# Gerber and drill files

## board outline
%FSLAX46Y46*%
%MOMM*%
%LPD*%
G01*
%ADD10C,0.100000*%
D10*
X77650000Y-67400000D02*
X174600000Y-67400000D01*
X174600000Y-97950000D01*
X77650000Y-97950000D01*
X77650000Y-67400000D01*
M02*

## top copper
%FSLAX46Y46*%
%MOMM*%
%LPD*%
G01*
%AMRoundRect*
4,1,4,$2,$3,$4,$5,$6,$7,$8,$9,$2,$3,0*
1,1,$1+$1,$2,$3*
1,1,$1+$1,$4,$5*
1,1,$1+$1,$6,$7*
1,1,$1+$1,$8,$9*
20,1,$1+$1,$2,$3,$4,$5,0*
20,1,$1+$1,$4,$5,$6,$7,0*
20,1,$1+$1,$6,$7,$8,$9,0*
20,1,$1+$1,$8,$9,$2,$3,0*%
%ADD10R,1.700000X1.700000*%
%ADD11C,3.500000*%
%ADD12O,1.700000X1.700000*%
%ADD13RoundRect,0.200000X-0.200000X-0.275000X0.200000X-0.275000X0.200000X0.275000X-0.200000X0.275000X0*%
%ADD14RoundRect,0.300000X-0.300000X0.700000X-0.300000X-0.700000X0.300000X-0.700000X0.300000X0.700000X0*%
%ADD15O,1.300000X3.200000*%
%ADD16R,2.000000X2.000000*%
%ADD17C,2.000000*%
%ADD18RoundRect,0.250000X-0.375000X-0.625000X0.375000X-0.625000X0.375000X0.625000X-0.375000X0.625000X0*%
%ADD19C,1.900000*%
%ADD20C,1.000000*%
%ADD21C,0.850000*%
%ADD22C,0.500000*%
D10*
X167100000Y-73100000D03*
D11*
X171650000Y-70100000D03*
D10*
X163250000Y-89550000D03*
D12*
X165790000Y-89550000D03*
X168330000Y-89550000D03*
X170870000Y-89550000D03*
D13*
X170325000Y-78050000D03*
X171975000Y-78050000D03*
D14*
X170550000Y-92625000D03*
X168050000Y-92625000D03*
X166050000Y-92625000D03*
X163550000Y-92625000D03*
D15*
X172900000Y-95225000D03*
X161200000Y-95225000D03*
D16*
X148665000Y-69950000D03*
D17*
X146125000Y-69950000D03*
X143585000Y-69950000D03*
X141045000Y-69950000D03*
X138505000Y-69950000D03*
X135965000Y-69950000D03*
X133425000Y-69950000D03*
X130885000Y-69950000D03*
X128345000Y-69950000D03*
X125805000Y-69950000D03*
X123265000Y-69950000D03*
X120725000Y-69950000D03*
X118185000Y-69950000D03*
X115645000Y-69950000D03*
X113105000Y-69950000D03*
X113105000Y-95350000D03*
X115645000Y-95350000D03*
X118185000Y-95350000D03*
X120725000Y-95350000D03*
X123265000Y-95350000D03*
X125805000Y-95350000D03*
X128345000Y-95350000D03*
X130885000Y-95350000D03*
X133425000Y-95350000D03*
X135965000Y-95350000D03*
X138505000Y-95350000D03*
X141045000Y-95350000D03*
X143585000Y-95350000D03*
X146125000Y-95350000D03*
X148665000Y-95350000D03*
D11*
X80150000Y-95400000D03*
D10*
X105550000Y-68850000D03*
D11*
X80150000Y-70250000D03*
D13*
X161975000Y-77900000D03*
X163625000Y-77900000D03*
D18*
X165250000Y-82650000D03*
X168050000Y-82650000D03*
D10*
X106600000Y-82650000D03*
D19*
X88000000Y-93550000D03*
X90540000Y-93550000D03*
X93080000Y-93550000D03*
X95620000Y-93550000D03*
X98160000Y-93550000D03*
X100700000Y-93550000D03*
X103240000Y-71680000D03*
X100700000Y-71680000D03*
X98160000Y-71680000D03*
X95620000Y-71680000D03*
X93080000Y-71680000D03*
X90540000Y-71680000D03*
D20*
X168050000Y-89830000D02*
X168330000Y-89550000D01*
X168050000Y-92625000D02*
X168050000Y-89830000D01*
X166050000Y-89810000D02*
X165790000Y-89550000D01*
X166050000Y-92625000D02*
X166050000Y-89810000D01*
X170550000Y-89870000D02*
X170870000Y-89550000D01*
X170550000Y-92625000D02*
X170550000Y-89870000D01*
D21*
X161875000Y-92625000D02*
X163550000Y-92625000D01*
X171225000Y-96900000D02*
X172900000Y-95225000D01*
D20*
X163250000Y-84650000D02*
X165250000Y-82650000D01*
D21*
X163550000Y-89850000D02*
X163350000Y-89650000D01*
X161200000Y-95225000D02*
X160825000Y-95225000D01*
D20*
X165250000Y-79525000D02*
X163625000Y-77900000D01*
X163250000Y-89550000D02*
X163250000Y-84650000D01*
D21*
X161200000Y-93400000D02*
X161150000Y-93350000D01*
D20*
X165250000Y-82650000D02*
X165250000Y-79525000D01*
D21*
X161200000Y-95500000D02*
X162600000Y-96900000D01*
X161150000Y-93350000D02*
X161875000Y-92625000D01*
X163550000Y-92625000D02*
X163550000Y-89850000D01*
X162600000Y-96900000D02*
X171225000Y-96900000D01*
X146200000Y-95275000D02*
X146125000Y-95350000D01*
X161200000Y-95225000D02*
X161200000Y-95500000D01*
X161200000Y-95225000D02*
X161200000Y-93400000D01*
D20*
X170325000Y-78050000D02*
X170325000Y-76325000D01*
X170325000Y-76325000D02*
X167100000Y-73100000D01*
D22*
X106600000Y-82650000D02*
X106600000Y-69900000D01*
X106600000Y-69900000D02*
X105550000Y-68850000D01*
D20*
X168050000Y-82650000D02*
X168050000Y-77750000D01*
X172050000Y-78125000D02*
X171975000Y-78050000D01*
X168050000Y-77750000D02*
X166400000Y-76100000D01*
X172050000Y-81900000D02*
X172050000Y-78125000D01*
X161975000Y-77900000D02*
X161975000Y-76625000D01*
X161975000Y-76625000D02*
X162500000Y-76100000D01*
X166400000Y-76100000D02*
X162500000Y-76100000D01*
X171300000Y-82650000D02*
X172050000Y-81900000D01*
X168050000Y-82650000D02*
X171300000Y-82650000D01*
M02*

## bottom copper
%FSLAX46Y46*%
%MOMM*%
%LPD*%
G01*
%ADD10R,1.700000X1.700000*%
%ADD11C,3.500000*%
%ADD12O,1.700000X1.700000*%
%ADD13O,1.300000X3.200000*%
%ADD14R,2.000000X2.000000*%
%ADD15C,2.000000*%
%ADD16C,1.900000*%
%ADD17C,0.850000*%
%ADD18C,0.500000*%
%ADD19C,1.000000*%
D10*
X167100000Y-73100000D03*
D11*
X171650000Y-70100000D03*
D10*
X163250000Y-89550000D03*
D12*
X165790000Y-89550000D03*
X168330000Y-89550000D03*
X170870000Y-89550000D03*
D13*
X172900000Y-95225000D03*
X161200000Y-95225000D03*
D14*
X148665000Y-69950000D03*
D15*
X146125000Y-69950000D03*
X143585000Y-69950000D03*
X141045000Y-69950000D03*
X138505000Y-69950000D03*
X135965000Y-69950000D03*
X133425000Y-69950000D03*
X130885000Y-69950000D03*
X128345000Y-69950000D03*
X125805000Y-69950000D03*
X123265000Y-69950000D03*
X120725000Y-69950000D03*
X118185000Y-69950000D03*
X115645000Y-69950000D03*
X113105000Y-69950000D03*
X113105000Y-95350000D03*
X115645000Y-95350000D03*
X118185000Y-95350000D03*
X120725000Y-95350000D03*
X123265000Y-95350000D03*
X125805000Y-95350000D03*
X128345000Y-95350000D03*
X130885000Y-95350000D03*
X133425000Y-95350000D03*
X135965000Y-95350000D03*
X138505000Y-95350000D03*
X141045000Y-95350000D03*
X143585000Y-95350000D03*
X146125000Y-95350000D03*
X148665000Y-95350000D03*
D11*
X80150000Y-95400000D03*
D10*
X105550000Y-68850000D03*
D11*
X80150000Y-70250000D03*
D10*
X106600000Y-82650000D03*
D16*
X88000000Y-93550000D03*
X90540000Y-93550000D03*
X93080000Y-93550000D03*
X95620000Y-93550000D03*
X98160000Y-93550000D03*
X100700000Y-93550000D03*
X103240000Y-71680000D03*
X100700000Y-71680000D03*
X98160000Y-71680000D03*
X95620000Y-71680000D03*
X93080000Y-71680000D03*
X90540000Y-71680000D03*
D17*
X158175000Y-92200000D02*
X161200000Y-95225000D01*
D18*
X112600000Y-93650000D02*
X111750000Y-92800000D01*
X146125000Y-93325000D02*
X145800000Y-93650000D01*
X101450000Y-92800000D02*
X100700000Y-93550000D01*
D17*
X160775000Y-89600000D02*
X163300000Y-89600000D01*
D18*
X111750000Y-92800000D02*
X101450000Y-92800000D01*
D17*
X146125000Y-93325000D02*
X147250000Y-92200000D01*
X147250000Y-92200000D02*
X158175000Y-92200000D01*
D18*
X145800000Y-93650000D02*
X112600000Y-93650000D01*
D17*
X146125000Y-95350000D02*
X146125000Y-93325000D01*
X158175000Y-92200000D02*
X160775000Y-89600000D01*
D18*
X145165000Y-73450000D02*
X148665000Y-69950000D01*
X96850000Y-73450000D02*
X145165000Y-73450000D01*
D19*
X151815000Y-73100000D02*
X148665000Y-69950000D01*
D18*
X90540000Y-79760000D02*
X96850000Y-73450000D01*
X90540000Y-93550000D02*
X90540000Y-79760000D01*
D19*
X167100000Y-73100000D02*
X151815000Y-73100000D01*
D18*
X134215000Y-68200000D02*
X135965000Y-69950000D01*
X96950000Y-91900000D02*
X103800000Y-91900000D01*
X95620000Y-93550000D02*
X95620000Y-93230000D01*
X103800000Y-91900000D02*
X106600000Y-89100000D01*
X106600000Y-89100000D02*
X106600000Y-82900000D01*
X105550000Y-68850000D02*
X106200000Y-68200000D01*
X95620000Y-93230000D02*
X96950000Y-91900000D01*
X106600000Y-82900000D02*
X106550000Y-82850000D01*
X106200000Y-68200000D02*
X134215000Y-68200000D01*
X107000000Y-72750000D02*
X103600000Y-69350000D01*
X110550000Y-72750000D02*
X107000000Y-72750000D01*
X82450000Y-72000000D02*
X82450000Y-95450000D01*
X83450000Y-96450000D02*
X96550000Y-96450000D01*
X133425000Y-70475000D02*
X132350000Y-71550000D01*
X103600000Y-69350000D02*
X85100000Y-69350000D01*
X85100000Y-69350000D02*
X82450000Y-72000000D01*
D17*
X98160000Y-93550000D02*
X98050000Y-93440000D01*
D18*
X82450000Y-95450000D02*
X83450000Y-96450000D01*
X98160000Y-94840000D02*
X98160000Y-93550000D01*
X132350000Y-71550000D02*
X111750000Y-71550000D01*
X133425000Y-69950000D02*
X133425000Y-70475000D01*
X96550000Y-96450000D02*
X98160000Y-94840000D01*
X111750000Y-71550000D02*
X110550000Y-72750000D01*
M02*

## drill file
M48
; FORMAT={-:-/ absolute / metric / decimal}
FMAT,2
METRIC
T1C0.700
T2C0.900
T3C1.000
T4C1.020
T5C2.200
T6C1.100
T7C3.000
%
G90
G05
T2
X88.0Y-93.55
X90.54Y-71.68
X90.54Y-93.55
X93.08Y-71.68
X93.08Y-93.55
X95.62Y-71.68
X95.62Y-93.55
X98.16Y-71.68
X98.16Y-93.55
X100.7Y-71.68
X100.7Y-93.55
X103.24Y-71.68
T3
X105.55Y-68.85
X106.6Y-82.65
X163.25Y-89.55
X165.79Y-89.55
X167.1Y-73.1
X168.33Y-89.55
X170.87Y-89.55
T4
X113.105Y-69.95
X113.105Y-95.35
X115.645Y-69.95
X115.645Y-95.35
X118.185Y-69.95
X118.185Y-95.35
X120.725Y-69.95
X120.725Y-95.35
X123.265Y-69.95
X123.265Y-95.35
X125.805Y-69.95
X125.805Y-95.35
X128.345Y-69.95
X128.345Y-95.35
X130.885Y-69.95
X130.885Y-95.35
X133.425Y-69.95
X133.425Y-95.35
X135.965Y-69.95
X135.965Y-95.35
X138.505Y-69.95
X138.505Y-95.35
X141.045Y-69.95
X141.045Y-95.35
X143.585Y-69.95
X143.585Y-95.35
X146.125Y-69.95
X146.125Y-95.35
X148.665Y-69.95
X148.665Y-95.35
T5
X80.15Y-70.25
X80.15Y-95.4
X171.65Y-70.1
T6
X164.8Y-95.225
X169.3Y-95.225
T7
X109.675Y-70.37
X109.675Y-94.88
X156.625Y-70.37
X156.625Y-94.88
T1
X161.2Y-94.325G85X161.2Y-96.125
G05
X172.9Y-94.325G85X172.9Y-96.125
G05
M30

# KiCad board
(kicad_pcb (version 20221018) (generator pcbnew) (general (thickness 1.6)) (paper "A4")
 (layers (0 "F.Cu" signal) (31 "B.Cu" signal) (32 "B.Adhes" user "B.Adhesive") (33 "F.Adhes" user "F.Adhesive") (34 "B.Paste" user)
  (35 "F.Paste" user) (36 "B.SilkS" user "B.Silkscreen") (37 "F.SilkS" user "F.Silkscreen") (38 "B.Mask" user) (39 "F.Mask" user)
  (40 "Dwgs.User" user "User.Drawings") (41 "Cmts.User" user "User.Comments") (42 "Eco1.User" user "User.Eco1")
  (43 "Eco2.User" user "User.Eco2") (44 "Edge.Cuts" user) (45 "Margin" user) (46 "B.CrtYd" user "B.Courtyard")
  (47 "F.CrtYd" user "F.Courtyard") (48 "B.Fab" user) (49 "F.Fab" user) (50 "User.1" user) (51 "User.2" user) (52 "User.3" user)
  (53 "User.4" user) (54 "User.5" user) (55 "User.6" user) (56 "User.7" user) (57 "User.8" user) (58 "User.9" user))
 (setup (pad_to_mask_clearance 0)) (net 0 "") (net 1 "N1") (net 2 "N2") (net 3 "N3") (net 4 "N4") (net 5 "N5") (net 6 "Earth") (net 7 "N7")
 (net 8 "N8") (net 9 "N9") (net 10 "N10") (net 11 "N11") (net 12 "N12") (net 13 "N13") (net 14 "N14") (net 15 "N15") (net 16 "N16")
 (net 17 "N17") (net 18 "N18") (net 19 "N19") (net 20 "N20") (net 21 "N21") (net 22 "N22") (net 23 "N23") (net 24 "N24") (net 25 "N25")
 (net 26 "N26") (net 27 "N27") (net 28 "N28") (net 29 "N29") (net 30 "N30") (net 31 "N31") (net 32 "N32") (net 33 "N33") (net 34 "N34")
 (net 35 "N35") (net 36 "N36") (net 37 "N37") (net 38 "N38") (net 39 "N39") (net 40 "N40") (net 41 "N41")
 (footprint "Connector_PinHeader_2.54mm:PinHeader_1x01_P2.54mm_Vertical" (layer "F.Cu") (at 167.1 73.1)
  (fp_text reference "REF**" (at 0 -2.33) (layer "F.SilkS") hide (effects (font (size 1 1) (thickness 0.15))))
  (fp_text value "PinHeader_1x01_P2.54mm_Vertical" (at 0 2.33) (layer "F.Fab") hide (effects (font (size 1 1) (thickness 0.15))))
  (pad "1" thru_hole rect (at 0 0) (size 1.7 1.7) (drill 1) (layers "*.Cu" "*.Mask")))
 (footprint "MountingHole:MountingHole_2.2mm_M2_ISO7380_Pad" (layer "F.Cu") (at 171.65 70.1)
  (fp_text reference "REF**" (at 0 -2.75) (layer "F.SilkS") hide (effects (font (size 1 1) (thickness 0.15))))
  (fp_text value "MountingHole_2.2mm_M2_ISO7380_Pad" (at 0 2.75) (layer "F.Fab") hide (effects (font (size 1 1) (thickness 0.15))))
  (pad "1" thru_hole circle (at 0 0) (size 3.5 3.5) (drill 2.2) (layers "*.Cu" "*.Mask")))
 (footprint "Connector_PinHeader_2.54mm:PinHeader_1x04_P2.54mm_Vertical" (layer "F.Cu") (at 163.25 89.55 90)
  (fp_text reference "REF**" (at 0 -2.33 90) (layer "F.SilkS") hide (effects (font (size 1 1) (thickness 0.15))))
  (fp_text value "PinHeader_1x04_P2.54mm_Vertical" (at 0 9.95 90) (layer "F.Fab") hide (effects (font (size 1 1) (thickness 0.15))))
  (pad "1" thru_hole rect (at 0 0 90) (size 1.7 1.7) (drill 1) (layers "*.Cu" "*.Mask"))
  (pad "2" thru_hole oval (at 0 2.54 90) (size 1.7 1.7) (drill 1) (layers "*.Cu" "*.Mask"))
  (pad "3" thru_hole oval (at 0 5.08 90) (size 1.7 1.7) (drill 1) (layers "*.Cu" "*.Mask"))
  (pad "4" thru_hole oval (at 0 7.62 90) (size 1.7 1.7) (drill 1) (layers "*.Cu" "*.Mask")))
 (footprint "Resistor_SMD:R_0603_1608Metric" (layer "F.Cu") (at 171.15 78.05)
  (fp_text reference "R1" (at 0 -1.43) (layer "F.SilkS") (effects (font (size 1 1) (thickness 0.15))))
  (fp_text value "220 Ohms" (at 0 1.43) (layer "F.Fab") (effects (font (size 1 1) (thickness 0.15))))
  (pad "1" smd roundrect (at -0.825 0) (size 0.8 0.95) (layers "F.Cu" "F.Paste" "F.Mask") (roundrect_rratio 0.25) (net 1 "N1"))
  (pad "2" smd roundrect (at 0.825 0) (size 0.8 0.95) (layers "F.Cu" "F.Paste" "F.Mask") (roundrect_rratio 0.25) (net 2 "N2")))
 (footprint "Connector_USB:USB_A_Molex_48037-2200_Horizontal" (layer "F.Cu") (at 167.05 103.6 -90)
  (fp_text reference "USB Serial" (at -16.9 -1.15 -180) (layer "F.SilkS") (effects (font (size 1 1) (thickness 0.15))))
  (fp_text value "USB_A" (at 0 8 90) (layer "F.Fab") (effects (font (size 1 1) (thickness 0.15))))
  (pad "" np_thru_hole circle (at -8.375 -2.25 270) (size 1.1 1.1) (drill 1.1) (layers "*.Mask"))
  (pad "" np_thru_hole circle (at -8.375 2.25 270) (size 1.1 1.1) (drill 1.1) (layers "*.Mask"))
  (pad "1" smd roundrect (at -10.975 -3.5 270) (size 2 1.2) (layers "F.Cu" "F.Paste" "F.Mask") (roundrect_rratio 0.25) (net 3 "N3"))
  (pad "2" smd roundrect (at -10.975 -1 270) (size 2 1.2) (layers "F.Cu" "F.Paste" "F.Mask") (roundrect_rratio 0.25) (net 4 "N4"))
  (pad "3" smd roundrect (at -10.975 1 270) (size 2 1.2) (layers "F.Cu" "F.Paste" "F.Mask") (roundrect_rratio 0.25) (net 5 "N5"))
  (pad "4" smd roundrect (at -10.975 3.5 270) (size 2 1.2) (layers "F.Cu" "F.Paste" "F.Mask") (roundrect_rratio 0.25) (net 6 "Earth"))
  (pad "5" thru_hole oval (at -8.375 -5.85 270) (size 3.2 1.3) (drill oval 2.5 0.7) (layers "*.Cu" "*.Mask") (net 6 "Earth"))
  (pad "5" thru_hole oval (at -8.375 5.85 270) (size 3.2 1.3) (drill oval 2.5 0.7) (layers "*.Cu" "*.Mask") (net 6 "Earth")))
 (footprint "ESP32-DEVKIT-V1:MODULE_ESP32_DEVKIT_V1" (layer "F.Cu") (at 133.15 82.65 -90)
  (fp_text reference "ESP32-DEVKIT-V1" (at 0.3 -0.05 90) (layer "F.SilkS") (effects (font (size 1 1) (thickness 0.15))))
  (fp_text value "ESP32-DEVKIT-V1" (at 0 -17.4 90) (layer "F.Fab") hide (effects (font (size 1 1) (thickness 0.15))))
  (pad "" np_thru_hole circle (at -12.28 -23.475 270) (size 3 3) (drill 3) (layers "*.Cu" "*.Mask"))
  (pad "" np_thru_hole circle (at -12.28 23.475 270) (size 3 3) (drill 3) (layers "*.Cu" "*.Mask"))
  (pad "" np_thru_hole circle (at 12.23 -23.475 270) (size 3 3) (drill 3) (layers "*.Cu" "*.Mask"))
  (pad "" np_thru_hole circle (at 12.23 23.475 270) (size 3 3) (drill 3) (layers "*.Cu" "*.Mask"))
  (pad "1" thru_hole rect (at -12.7 -15.515 270) (size 2 2) (drill 1.02) (layers "*.Cu" "*.Mask") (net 1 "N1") (solder_mask_margin 0.102))
  (pad "2" thru_hole circle (at -12.7 -12.975 270) (size 2 2) (drill 1.02) (layers "*.Cu" "*.Mask") (solder_mask_margin 0.102))
  (pad "3" thru_hole circle (at -12.7 -10.435 270) (size 2 2) (drill 1.02) (layers "*.Cu" "*.Mask") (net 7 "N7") (solder_mask_margin 0.102))
  (pad "4" thru_hole circle (at -12.7 -7.895 270) (size 2 2) (drill 1.02) (layers "*.Cu" "*.Mask") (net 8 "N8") (solder_mask_margin 0.102))
  (pad "5" thru_hole circle (at -12.7 -5.355 270) (size 2 2) (drill 1.02) (layers "*.Cu" "*.Mask") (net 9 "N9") (solder_mask_margin 0.102))
  (pad "6" thru_hole circle (at -12.7 -2.815 270) (size 2 2) (drill 1.02) (layers "*.Cu" "*.Mask") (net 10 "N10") (solder_mask_margin 0.102))
  (pad "7" thru_hole circle (at -12.7 -0.275 270) (size 2 2) (drill 1.02) (layers "*.Cu" "*.Mask") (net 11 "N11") (solder_mask_margin 0.102))
  (pad "8" thru_hole circle (at -12.7 2.265 270) (size 2 2) (drill 1.02) (layers "*.Cu" "*.Mask") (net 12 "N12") (solder_mask_margin 0.102))
  (pad "9" thru_hole circle (at -12.7 4.805 270) (size 2 2) (drill 1.02) (layers "*.Cu" "*.Mask") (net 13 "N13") (solder_mask_margin 0.102))
  (pad "10" thru_hole circle (at -12.7 7.345 270) (size 2 2) (drill 1.02) (layers "*.Cu" "*.Mask") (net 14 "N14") (solder_mask_margin 0.102))
  (pad "11" thru_hole circle (at -12.7 9.885 270) (size 2 2) (drill 1.02) (layers "*.Cu" "*.Mask") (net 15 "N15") (solder_mask_margin 0.102))
  (pad "12" thru_hole circle (at -12.7 12.425 270) (size 2 2) (drill 1.02) (layers "*.Cu" "*.Mask") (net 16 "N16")
   (solder_mask_margin 0.102))
  (pad "13" thru_hole circle (at -12.7 14.965 270) (size 2 2) (drill 1.02) (layers "*.Cu" "*.Mask") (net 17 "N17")
   (solder_mask_margin 0.102))
  (pad "14" thru_hole circle (at -12.7 17.505 270) (size 2 2) (drill 1.02) (layers "*.Cu" "*.Mask") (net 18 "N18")
   (solder_mask_margin 0.102))
  (pad "15" thru_hole circle (at -12.7 20.045 270) (size 2 2) (drill 1.02) (layers "*.Cu" "*.Mask") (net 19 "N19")
   (solder_mask_margin 0.102))
  (pad "16" thru_hole circle (at 12.7 20.045 270) (size 2 2) (drill 1.02) (layers "*.Cu" "*.Mask") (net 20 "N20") (solder_mask_margin 0.102))
  (pad "17" thru_hole circle (at 12.7 17.505 270) (size 2 2) (drill 1.02) (layers "*.Cu" "*.Mask") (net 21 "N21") (solder_mask_margin 0.102))
  (pad "18" thru_hole circle (at 12.7 14.965 270) (size 2 2) (drill 1.02) (layers "*.Cu" "*.Mask") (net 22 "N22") (solder_mask_margin 0.102))
  (pad "19" thru_hole circle (at 12.7 12.425 270) (size 2 2) (drill 1.02) (layers "*.Cu" "*.Mask") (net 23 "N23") (solder_mask_margin 0.102))
  (pad "20" thru_hole circle (at 12.7 9.885 270) (size 2 2) (drill 1.02) (layers "*.Cu" "*.Mask") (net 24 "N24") (solder_mask_margin 0.102))
  (pad "21" thru_hole circle (at 12.7 7.345 270) (size 2 2) (drill 1.02) (layers "*.Cu" "*.Mask") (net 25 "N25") (solder_mask_margin 0.102))
  (pad "22" thru_hole circle (at 12.7 4.805 270) (size 2 2) (drill 1.02) (layers "*.Cu" "*.Mask") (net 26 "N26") (solder_mask_margin 0.102))
  (pad "23" thru_hole circle (at 12.7 2.265 270) (size 2 2) (drill 1.02) (layers "*.Cu" "*.Mask") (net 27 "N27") (solder_mask_margin 0.102))
  (pad "24" thru_hole circle (at 12.7 -0.275 270) (size 2 2) (drill 1.02) (layers "*.Cu" "*.Mask") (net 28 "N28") (solder_mask_margin 0.102))
  (pad "25" thru_hole circle (at 12.7 -2.815 270) (size 2 2) (drill 1.02) (layers "*.Cu" "*.Mask") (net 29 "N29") (solder_mask_margin 0.102))
  (pad "26" thru_hole circle (at 12.7 -5.355 270) (size 2 2) (drill 1.02) (layers "*.Cu" "*.Mask") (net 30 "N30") (solder_mask_margin 0.102))
  (pad "27" thru_hole circle (at 12.7 -7.895 270) (size 2 2) (drill 1.02) (layers "*.Cu" "*.Mask") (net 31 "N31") (solder_mask_margin 0.102))
  (pad "28" thru_hole circle (at 12.7 -10.435 270) (size 2 2) (drill 1.02) (layers "*.Cu" "*.Mask") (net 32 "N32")
   (solder_mask_margin 0.102))
  (pad "29" thru_hole circle (at 12.7 -12.975 270) (size 2 2) (drill 1.02) (layers "*.Cu" "*.Mask") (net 6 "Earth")
   (solder_mask_margin 0.102))
  (pad "30" thru_hole circle (at 12.7 -15.515 270) (size 2 2) (drill 1.02) (layers "*.Cu" "*.Mask") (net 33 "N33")
   (solder_mask_margin 0.102))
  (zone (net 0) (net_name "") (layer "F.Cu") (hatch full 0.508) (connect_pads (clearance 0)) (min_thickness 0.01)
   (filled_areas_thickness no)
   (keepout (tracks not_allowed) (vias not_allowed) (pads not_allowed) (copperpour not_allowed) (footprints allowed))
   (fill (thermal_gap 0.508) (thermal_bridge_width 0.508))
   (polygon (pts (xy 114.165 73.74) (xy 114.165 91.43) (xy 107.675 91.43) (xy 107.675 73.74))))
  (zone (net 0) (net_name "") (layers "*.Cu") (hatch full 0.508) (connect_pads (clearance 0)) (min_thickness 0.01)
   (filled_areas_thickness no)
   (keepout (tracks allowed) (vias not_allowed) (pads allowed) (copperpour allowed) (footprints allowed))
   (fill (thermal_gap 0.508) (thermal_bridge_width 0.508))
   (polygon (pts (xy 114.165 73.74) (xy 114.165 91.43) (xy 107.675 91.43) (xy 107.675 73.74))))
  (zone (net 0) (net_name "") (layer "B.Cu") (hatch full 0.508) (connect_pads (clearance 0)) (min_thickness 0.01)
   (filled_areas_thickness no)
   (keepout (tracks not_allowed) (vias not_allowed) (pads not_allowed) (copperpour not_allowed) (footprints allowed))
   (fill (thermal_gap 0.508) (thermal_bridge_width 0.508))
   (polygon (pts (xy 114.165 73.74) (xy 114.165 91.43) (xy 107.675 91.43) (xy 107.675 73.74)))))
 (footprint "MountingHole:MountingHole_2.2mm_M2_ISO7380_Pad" (layer "F.Cu") (at 80.15 95.4)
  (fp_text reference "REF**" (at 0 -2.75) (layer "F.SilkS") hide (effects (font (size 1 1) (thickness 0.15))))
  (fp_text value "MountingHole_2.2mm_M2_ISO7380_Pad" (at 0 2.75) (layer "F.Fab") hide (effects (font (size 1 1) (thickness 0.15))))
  (pad "1" thru_hole circle (at 0 0) (size 3.5 3.5) (drill 2.2) (layers "*.Cu" "*.Mask")))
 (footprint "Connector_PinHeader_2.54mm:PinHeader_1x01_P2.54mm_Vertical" (layer "F.Cu") (at 105.55 68.85)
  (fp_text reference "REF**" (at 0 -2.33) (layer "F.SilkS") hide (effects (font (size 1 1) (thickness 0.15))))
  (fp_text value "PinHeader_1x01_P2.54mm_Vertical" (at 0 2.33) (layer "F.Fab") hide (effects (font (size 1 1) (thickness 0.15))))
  (pad "1" thru_hole rect (at 0 0) (size 1.7 1.7) (drill 1) (layers "*.Cu" "*.Mask")))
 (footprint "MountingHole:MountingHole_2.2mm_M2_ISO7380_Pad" (layer "F.Cu") (at 80.15 70.25)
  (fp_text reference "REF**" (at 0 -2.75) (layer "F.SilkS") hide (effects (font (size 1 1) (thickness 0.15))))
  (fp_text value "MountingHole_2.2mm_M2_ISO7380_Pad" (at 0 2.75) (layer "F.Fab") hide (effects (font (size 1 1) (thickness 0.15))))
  (pad "1" thru_hole circle (at 0 0) (size 3.5 3.5) (drill 2.2) (layers "*.Cu" "*.Mask")))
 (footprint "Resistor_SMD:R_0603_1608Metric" (layer "F.Cu") (at 162.8 77.9)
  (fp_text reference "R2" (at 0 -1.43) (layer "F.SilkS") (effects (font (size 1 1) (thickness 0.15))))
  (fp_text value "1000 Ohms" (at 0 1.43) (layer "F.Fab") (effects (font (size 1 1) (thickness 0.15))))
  (pad "1" smd roundrect (at -0.825 0) (size 0.8 0.95) (layers "F.Cu" "F.Paste" "F.Mask") (roundrect_rratio 0.25) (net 2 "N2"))
  (pad "2" smd roundrect (at 0.825 0) (size 0.8 0.95) (layers "F.Cu" "F.Paste" "F.Mask") (roundrect_rratio 0.25) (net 6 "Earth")))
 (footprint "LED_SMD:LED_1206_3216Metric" (layer "F.Cu") (at 166.65 82.65)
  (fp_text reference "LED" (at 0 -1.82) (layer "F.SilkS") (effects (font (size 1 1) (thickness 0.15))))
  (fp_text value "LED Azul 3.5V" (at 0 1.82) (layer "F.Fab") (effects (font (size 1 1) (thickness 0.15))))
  (pad "1" smd roundrect (at -1.4 0) (size 1.25 1.75) (layers "F.Cu" "F.Paste" "F.Mask") (roundrect_rratio 0.2) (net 6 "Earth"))
  (pad "2" smd roundrect (at 1.4 0) (size 1.25 1.75) (layers "F.Cu" "F.Paste" "F.Mask") (roundrect_rratio 0.2) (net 2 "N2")))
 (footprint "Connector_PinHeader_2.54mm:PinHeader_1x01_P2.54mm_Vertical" (layer "F.Cu") (at 106.6 82.65)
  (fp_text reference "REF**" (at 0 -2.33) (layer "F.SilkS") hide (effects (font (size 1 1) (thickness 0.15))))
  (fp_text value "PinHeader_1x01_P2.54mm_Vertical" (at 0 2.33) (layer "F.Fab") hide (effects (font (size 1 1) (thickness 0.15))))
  (pad "1" thru_hole rect (at 0 0) (size 1.7 1.7) (drill 1) (layers "*.Cu" "*.Mask")))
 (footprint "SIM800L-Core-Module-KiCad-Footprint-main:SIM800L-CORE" (layer "F.Cu") (at 88 93.55 90)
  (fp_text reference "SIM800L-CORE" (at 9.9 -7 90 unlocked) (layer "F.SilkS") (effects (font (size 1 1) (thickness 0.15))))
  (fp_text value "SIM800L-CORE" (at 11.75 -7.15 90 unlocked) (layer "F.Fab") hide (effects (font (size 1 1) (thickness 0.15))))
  (pad "1" thru_hole circle (at 0 0 90) (size 1.9 1.9) (drill 0.9) (layers "*.Cu" "*.Mask") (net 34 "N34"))
  (pad "2" thru_hole circle (at 0 2.54 90) (size 1.9 1.9) (drill 0.9) (layers "*.Cu" "*.Mask") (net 1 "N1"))
  (pad "3" thru_hole circle (at 0 5.08 90) (size 1.9 1.9) (drill 0.9) (layers "*.Cu" "*.Mask") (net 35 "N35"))
  (pad "4" thru_hole circle (at 0 7.62 90) (size 1.9 1.9) (drill 0.9) (layers "*.Cu" "*.Mask") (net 10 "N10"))
  (pad "5" thru_hole circle (at 0 10.16 90) (size 1.9 1.9) (drill 0.9) (layers "*.Cu" "*.Mask") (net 11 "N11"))
  (pad "6" thru_hole circle (at 0 12.7 90) (size 1.9 1.9) (drill 0.9) (layers "*.Cu" "*.Mask") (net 6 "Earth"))
  (pad "7" thru_hole circle (at 21.87 15.24 90) (size 1.9 1.9) (drill 0.9) (layers "*.Cu" "*.Mask") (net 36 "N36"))
  (pad "8" thru_hole circle (at 21.87 12.7 90) (size 1.9 1.9) (drill 0.9) (layers "*.Cu" "*.Mask") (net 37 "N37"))
  (pad "9" thru_hole circle (at 21.87 10.16 90) (size 1.9 1.9) (drill 0.9) (layers "*.Cu" "*.Mask") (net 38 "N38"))
  (pad "10" thru_hole circle (at 21.87 7.62 90) (size 1.9 1.9) (drill 0.9) (layers "*.Cu" "*.Mask") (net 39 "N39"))
  (pad "11" thru_hole circle (at 21.87 5.08 90) (size 1.9 1.9) (drill 0.9) (layers "*.Cu" "*.Mask") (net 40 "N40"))
  (pad "12" thru_hole circle (at 21.87 2.54 90) (size 1.9 1.9) (drill 0.9) (layers "*.Cu" "*.Mask") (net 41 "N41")))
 (gr_rect locked (start 77.65 67.4) (end 174.6 97.95) (stroke (width 0.1) (type default)) (fill none) (layer "Edge.Cuts"))
 (segment (start 168.05 89.83) (end 168.33 89.55) (width 1) (layer "F.Cu") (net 4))
 (segment (start 168.05 92.625) (end 168.05 89.83) (width 1) (layer "F.Cu") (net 4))
 (segment (start 166.05 89.81) (end 165.79 89.55) (width 1) (layer "F.Cu") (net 5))
 (segment (start 166.05 92.625) (end 166.05 89.81) (width 1) (layer "F.Cu") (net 5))
 (segment (start 170.55 89.87) (end 170.87 89.55) (width 1) (layer "F.Cu") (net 3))
 (segment (start 170.55 92.625) (end 170.55 89.87) (width 1) (layer "F.Cu") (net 3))
 (segment (start 161.875 92.625) (end 163.55 92.625) (width 0.85) (layer "F.Cu") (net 6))
 (segment (start 171.225 96.9) (end 172.9 95.225) (width 0.85) (layer "F.Cu") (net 6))
 (segment (start 163.25 84.65) (end 165.25 82.65) (width 1) (layer "F.Cu") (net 6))
 (segment (start 163.55 89.85) (end 163.35 89.65) (width 0.85) (layer "F.Cu") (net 6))
 (segment (start 161.2 95.225) (end 160.825 95.225) (width 0.85) (layer "F.Cu") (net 6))
 (segment (start 165.25 79.525) (end 163.625 77.9) (width 1) (layer "F.Cu") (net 6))
 (segment (start 163.25 89.55) (end 163.25 84.65) (width 1) (layer "F.Cu") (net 6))
 (segment (start 161.2 93.4) (end 161.15 93.35) (width 0.85) (layer "F.Cu") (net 6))
 (segment (start 165.25 82.65) (end 165.25 79.525) (width 1) (layer "F.Cu") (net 6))
 (segment (start 161.2 95.5) (end 162.6 96.9) (width 0.85) (layer "F.Cu") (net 6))
 (segment (start 161.15 93.35) (end 161.875 92.625) (width 0.85) (layer "F.Cu") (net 6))
 (segment (start 163.55 92.625) (end 163.55 89.85) (width 0.85) (layer "F.Cu") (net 6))
 (segment (start 162.6 96.9) (end 171.225 96.9) (width 0.85) (layer "F.Cu") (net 6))
 (segment (start 146.2 95.275) (end 146.125 95.35) (width 0.85) (layer "F.Cu") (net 6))
 (segment (start 161.2 95.225) (end 161.2 95.5) (width 0.85) (layer "F.Cu") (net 6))
 (segment (start 161.2 95.225) (end 161.2 93.4) (width 0.85) (layer "F.Cu") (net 6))
 (segment (start 158.175 92.2) (end 161.2 95.225) (width 0.85) (layer "B.Cu") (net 6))
 (segment (start 112.6 93.65) (end 111.75 92.8) (width 0.5) (layer "B.Cu") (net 6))
 (segment (start 146.125 93.325) (end 145.8 93.65) (width 0.5) (layer "B.Cu") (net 6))
 (segment (start 101.45 92.8) (end 100.7 93.55) (width 0.5) (layer "B.Cu") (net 6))
 (segment (start 160.775 89.6) (end 163.3 89.6) (width 0.85) (layer "B.Cu") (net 6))
 (segment (start 111.75 92.8) (end 101.45 92.8) (width 0.5) (layer "B.Cu") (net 6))
 (segment (start 146.125 93.325) (end 147.25 92.2) (width 0.85) (layer "B.Cu") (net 6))
 (segment (start 147.25 92.2) (end 158.175 92.2) (width 0.85) (layer "B.Cu") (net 6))
 (segment (start 145.8 93.65) (end 112.6 93.65) (width 0.5) (layer "B.Cu") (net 6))
 (segment (start 146.125 95.35) (end 146.125 93.325) (width 0.85) (layer "B.Cu") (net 6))
 (segment (start 158.175 92.2) (end 160.775 89.6) (width 0.85) (layer "B.Cu") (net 6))
 (segment (start 170.325 78.05) (end 170.325 76.325) (width 1) (layer "F.Cu") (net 1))
 (segment (start 170.325 76.325) (end 167.1 73.1) (width 1) (layer "F.Cu") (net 1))
 (segment (start 145.165 73.45) (end 148.665 69.95) (width 0.5) (layer "B.Cu") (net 1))
 (segment (start 96.85 73.45) (end 145.165 73.45) (width 0.5) (layer "B.Cu") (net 1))
 (segment (start 151.815 73.1) (end 148.665 69.95) (width 1) (layer "B.Cu") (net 1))
 (segment (start 90.54 79.76) (end 96.85 73.45) (width 0.5) (layer "B.Cu") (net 1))
 (segment (start 90.54 93.55) (end 90.54 79.76) (width 0.5) (layer "B.Cu") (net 1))
 (segment (start 167.1 73.1) (end 151.815 73.1) (width 1) (layer "B.Cu") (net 1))
 (segment (start 106.6 82.65) (end 106.6 69.9) (width 0.5) (layer "F.Cu") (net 10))
 (segment (start 106.6 69.9) (end 105.55 68.85) (width 0.5) (layer "F.Cu") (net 10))
 (segment (start 134.215 68.2) (end 135.965 69.95) (width 0.5) (layer "B.Cu") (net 10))
 (segment (start 96.95 91.9) (end 103.8 91.9) (width 0.5) (layer "B.Cu") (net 10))
 (segment (start 95.62 93.55) (end 95.62 93.23) (width 0.5) (layer "B.Cu") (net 10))
 (segment (start 103.8 91.9) (end 106.6 89.1) (width 0.5) (layer "B.Cu") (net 10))
 (segment (start 106.6 89.1) (end 106.6 82.9) (width 0.5) (layer "B.Cu") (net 10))
 (segment (start 105.55 68.85) (end 106.2 68.2) (width 0.5) (layer "B.Cu") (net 10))
 (segment (start 95.62 93.23) (end 96.95 91.9) (width 0.5) (layer "B.Cu") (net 10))
 (segment (start 106.6 82.9) (end 106.55 82.85) (width 0.5) (layer "B.Cu") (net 10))
 (segment (start 106.2 68.2) (end 134.215 68.2) (width 0.5) (layer "B.Cu") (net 10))
 (segment (start 107 72.75) (end 103.6 69.35) (width 0.5) (layer "B.Cu") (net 11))
 (segment (start 110.55 72.75) (end 107 72.75) (width 0.5) (layer "B.Cu") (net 11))
 (segment (start 82.45 72) (end 82.45 95.45) (width 0.5) (layer "B.Cu") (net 11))
 (segment (start 83.45 96.45) (end 96.55 96.45) (width 0.5) (layer "B.Cu") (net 11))
 (segment (start 133.425 70.475) (end 132.35 71.55) (width 0.5) (layer "B.Cu") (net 11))
 (segment (start 103.6 69.35) (end 85.1 69.35) (width 0.5) (layer "B.Cu") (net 11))
 (segment (start 85.1 69.35) (end 82.45 72) (width 0.5) (layer "B.Cu") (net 11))
 (segment (start 98.16 93.55) (end 98.05 93.44) (width 0.85) (layer "B.Cu") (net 11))
 (segment (start 82.45 95.45) (end 83.45 96.45) (width 0.5) (layer "B.Cu") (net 11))
 (segment (start 98.16 94.84) (end 98.16 93.55) (width 0.5) (layer "B.Cu") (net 11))
 (segment (start 132.35 71.55) (end 111.75 71.55) (width 0.5) (layer "B.Cu") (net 11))
 (segment (start 133.425 69.95) (end 133.425 70.475) (width 0.5) (layer "B.Cu") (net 11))
 (segment (start 96.55 96.45) (end 98.16 94.84) (width 0.5) (layer "B.Cu") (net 11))
 (segment (start 111.75 71.55) (end 110.55 72.75) (width 0.5) (layer "B.Cu") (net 11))
 (segment (start 168.05 82.65) (end 168.05 77.75) (width 1) (layer "F.Cu") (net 2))
 (segment (start 172.05 78.125) (end 171.975 78.05) (width 1) (layer "F.Cu") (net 2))
 (segment (start 168.05 77.75) (end 166.4 76.1) (width 1) (layer "F.Cu") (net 2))
 (segment (start 172.05 81.9) (end 172.05 78.125) (width 1) (layer "F.Cu") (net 2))
 (segment (start 161.975 77.9) (end 161.975 76.625) (width 1) (layer "F.Cu") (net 2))
 (segment (start 161.975 76.625) (end 162.5 76.1) (width 1) (layer "F.Cu") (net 2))
 (segment (start 166.4 76.1) (end 162.5 76.1) (width 1) (layer "F.Cu") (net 2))
 (segment (start 171.3 82.65) (end 172.05 81.9) (width 1) (layer "F.Cu") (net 2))
 (segment (start 168.05 82.65) (end 171.3 82.65) (width 1) (layer "F.Cu") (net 2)))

